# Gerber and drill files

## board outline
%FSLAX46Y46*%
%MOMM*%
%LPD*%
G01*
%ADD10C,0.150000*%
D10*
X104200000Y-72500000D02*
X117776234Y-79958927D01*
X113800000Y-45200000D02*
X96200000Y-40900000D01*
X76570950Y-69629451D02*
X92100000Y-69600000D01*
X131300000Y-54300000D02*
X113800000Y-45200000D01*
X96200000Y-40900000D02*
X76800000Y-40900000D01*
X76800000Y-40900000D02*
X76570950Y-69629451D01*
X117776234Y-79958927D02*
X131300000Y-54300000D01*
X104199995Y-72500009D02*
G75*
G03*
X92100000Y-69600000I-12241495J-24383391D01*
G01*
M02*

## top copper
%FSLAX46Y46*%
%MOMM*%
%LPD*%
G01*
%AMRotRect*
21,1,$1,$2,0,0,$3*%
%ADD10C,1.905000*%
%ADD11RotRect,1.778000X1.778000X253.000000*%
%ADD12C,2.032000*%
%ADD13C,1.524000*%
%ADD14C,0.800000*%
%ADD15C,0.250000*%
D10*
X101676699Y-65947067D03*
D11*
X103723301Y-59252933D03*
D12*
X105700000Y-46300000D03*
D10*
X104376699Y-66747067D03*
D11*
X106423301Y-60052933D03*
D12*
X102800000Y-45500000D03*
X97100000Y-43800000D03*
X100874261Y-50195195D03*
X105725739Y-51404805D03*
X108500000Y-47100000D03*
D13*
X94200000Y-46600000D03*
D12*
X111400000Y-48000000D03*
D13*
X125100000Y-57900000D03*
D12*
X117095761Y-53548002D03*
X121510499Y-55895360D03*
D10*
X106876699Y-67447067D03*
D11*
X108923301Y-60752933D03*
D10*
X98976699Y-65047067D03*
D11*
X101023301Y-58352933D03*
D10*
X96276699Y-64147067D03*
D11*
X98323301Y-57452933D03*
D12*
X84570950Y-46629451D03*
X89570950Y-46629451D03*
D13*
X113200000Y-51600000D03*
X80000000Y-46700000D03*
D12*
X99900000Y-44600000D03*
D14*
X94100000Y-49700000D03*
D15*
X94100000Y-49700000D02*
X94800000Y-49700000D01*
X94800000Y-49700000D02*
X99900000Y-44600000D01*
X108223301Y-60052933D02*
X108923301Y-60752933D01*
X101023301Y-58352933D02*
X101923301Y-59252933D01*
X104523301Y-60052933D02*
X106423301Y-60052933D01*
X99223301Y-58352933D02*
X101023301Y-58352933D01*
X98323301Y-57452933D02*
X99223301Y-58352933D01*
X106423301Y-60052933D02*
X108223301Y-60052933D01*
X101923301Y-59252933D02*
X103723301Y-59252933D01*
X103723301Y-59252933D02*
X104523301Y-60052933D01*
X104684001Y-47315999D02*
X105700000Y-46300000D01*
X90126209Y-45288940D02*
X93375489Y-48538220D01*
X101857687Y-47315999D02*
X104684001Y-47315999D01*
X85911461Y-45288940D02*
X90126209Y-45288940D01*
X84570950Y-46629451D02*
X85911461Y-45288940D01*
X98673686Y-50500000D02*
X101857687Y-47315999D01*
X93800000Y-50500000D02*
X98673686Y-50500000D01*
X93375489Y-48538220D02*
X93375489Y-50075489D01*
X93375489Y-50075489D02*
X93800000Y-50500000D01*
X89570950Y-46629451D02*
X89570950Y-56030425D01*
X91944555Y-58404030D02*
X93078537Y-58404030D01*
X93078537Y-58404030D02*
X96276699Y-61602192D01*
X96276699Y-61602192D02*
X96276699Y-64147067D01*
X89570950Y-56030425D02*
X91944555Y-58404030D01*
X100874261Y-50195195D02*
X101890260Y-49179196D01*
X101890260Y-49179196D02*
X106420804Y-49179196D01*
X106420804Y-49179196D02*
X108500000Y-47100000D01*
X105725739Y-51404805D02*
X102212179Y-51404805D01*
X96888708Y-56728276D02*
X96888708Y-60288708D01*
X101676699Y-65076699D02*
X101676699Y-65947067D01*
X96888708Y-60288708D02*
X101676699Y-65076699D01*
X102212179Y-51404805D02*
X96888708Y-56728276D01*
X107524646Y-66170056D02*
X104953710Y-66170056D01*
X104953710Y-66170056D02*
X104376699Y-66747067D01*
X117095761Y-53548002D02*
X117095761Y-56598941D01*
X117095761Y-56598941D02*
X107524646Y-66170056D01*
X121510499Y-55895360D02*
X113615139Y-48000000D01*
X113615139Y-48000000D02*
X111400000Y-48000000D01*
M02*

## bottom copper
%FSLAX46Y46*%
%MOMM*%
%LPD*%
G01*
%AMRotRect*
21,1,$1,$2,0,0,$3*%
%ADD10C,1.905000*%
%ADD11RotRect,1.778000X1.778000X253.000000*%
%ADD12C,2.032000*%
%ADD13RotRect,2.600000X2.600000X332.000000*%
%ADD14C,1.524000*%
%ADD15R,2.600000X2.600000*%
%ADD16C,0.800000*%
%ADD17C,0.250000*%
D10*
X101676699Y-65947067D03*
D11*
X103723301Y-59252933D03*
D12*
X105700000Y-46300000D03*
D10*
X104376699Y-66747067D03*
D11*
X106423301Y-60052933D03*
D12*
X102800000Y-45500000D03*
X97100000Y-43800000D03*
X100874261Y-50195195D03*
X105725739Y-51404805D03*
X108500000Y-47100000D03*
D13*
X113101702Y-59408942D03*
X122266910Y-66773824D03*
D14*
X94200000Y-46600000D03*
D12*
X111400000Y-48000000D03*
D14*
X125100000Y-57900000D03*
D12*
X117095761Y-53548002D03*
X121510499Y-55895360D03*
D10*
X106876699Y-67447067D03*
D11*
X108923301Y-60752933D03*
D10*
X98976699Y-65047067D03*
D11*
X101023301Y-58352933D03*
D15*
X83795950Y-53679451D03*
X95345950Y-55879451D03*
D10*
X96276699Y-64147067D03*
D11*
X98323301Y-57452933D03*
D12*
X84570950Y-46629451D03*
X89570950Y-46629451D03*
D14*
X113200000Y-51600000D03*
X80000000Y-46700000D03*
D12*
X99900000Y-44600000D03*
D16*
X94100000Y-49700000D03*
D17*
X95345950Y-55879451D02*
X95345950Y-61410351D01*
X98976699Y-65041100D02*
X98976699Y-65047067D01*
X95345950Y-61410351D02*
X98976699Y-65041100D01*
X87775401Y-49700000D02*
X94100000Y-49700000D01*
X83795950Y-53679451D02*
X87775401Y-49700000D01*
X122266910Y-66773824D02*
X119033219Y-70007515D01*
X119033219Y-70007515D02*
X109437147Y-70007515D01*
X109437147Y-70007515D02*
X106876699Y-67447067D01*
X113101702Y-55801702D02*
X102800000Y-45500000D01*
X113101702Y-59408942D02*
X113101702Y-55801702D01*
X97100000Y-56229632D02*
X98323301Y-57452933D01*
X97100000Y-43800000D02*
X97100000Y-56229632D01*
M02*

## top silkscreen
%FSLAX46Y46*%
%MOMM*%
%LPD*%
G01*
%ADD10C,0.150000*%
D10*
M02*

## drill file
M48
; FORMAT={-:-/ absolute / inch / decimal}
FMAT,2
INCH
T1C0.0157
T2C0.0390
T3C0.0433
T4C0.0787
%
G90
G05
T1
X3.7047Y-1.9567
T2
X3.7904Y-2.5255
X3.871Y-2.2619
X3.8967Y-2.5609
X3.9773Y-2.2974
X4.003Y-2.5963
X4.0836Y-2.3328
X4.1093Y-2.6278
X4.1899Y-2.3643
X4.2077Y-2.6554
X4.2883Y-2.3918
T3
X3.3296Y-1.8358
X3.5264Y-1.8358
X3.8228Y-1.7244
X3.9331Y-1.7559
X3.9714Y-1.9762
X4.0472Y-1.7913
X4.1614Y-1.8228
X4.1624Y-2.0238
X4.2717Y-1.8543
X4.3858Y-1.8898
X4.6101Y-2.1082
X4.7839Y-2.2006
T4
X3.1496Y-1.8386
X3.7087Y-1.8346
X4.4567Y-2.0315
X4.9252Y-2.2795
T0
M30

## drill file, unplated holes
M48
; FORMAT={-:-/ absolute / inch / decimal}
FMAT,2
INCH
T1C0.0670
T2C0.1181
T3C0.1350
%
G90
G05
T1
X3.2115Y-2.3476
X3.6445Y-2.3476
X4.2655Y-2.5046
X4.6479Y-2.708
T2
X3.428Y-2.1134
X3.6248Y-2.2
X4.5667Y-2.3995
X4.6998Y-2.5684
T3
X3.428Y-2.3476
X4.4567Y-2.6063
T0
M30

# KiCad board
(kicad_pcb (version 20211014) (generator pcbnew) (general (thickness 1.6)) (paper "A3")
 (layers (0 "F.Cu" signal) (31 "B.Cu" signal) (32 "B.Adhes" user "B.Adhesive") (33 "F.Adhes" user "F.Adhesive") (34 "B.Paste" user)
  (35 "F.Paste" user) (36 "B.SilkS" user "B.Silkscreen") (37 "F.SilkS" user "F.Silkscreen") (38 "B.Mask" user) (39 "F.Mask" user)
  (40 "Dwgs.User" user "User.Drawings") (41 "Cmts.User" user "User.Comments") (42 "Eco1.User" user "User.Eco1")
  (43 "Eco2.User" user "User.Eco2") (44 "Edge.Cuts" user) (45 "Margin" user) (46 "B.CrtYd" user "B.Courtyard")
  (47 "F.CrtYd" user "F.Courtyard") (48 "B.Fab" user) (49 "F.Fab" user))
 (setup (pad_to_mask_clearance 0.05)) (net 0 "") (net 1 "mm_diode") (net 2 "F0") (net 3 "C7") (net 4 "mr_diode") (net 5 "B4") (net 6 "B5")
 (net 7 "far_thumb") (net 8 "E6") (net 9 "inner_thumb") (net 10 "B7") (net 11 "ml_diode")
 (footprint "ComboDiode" (layer "F.Cu") (at 102.7 62.6 -107)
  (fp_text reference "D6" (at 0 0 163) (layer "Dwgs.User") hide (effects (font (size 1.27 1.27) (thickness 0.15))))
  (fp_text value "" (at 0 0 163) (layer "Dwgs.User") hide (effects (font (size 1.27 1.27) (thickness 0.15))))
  (pad "1" thru_hole circle locked (at 3.5 0 253) (size 1.905 1.905) (drill 0.9906) (layers *.Cu *.Mask) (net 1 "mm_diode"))
  (pad "2" thru_hole rect locked (at -3.5 0 253) (size 1.778 1.778) (drill 0.9906) (layers *.Cu *.Mask) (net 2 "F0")))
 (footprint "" (layer "F.Cu") (at 105.7 46.3)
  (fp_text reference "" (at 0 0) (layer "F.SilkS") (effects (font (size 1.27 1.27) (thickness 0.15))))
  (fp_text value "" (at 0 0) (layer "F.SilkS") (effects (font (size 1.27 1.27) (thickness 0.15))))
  (pad "1" thru_hole circle locked (at 0 0) (size 2.032 2.032) (drill 1.1) (layers *.Cu *.Mask) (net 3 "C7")))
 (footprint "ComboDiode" (layer "F.Cu") (at 105.4 63.4 -107)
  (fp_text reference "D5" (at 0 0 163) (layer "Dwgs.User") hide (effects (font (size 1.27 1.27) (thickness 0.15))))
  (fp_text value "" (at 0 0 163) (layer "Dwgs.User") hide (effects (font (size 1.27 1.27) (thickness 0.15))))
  (pad "1" thru_hole circle locked (at 3.5 0 253) (size 1.905 1.905) (drill 0.9906) (layers *.Cu *.Mask) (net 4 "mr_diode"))
  (pad "2" thru_hole rect locked (at -3.5 0 253) (size 1.778 1.778) (drill 0.9906) (layers *.Cu *.Mask) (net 2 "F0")))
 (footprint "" (layer "F.Cu") (at 102.8 45.5)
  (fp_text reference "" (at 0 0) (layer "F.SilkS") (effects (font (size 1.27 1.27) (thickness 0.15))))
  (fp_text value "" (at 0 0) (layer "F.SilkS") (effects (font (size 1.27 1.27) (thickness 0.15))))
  (pad "1" thru_hole circle locked (at 0 0) (size 2.032 2.032) (drill 1.1) (layers *.Cu *.Mask) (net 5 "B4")))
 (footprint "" (layer "F.Cu") (at 97.1 43.8)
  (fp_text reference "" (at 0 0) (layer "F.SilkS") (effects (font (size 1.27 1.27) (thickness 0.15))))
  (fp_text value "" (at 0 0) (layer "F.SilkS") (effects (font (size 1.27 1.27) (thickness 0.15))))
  (pad "1" thru_hole circle locked (at 0 0) (size 2.032 2.032) (drill 1.1) (layers *.Cu *.Mask) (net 2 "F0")))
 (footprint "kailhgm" (layer "F.Cu") (at 103.3 50.8 -14)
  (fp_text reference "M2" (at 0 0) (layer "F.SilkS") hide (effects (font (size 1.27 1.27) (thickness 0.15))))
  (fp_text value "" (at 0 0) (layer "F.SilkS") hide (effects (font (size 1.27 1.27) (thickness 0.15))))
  (pad "1" thru_hole circle locked (at -2.5 0) (size 2.032 2.032) (drill 1.1) (layers *.Cu *.Mask) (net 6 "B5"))
  (pad "2" thru_hole circle locked (at 2.5 0) (size 2.032 2.032) (drill 1.1) (layers *.Cu *.Mask) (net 1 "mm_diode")))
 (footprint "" (layer "F.Cu") (at 108.5 47.1)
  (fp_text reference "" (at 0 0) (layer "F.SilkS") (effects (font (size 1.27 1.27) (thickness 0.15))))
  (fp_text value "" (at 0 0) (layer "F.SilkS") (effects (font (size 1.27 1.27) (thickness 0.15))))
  (pad "1" thru_hole circle locked (at 0 0) (size 2.032 2.032) (drill 1.1) (layers *.Cu *.Mask) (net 6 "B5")))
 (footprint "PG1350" (layer "F.Cu") (at 113.2 66.2 -28)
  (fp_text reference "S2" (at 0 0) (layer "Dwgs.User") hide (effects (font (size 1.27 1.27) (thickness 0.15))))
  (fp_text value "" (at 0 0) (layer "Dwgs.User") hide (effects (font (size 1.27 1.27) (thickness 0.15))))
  (pad "" np_thru_hole circle locked (at 5 -3.75) (size 3 3) (drill 3) (layers *.Cu *.Mask))
  (pad "" np_thru_hole circle locked (at 5.5 0) (size 1.7018 1.7018) (drill 1.7018) (layers *.Cu *.Mask))
  (pad "" np_thru_hole circle locked (at 0 0) (size 3.429 3.429) (drill 3.429) (layers *.Cu *.Mask))
  (pad "" np_thru_hole circle locked (at -5.5 0) (size 1.7018 1.7018) (drill 1.7018) (layers *.Cu *.Mask))
  (pad "" np_thru_hole circle locked (at 0 -5.95) (size 3 3) (drill 3) (layers *.Cu *.Mask))
  (pad "1" smd rect locked (at -3.275 -5.95 332) (size 2.6 2.6) (layers "B.Cu" "B.Paste" "B.Mask") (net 5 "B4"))
  (pad "2" smd rect locked (at 8.275 -3.75 332) (size 2.6 2.6) (layers "B.Cu" "B.Paste" "B.Mask") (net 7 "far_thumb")))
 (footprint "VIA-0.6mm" (layer "F.Cu") (at 94.2 46.6)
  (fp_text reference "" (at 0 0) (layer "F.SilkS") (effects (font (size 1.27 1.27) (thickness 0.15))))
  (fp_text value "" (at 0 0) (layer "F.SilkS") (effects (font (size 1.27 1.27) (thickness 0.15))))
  (pad "1" thru_hole circle locked (at 0 0) (size 1.524 1.524) (drill 2) (layers *.Cu *.Mask)))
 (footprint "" (layer "F.Cu") (at 111.4 48)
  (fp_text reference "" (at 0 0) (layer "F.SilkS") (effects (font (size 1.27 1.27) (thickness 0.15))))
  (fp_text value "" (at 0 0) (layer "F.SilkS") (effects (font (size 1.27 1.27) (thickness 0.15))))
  (pad "1" thru_hole circle locked (at 0 0) (size 2.032 2.032) (drill 1.1) (layers *.Cu *.Mask) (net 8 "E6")))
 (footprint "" (layer "F.Cu") (at 125.1 57.9)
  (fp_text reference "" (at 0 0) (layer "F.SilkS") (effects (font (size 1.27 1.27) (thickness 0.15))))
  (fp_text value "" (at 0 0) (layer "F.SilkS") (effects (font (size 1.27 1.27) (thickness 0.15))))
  (pad "1" thru_hole circle locked (at 0 0) (size 1.524 1.524) (drill 2) (layers *.Cu *.Mask)))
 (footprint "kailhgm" (layer "F.Cu") (at 119.30313 54.721681 -28)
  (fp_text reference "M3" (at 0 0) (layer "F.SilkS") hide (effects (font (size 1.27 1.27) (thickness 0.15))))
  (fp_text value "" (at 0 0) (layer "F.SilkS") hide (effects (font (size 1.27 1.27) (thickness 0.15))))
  (pad "1" thru_hole circle locked (at -2.5 0) (size 2.032 2.032) (drill 1.1) (layers *.Cu *.Mask) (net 4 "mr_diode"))
  (pad "2" thru_hole circle locked (at 2.5 0) (size 2.032 2.032) (drill 1.1) (layers *.Cu *.Mask) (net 8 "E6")))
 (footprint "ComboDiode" (layer "F.Cu") (at 107.9 64.1 -107)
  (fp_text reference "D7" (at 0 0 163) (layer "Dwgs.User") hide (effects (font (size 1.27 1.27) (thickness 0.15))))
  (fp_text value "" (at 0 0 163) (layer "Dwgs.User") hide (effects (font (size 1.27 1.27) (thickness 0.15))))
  (pad "1" thru_hole circle locked (at 3.5 0 253) (size 1.905 1.905) (drill 0.9906) (layers *.Cu *.Mask) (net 7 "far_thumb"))
  (pad "2" thru_hole rect locked (at -3.5 0 253) (size 1.778 1.778) (drill 0.9906) (layers *.Cu *.Mask) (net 2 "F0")))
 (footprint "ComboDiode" (layer "F.Cu") (at 100 61.7 -107)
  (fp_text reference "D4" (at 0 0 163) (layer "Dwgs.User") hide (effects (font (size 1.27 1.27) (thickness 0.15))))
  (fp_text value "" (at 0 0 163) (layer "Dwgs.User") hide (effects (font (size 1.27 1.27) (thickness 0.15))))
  (pad "1" thru_hole circle locked (at 3.5 0 253) (size 1.905 1.905) (drill 0.9906) (layers *.Cu *.Mask) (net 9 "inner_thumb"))
  (pad "2" thru_hole rect locked (at -3.5 0 253) (size 1.778 1.778) (drill 0.9906) (layers *.Cu *.Mask) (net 2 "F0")))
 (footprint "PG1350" (layer "F.Cu") (at 87.07095 59.629451)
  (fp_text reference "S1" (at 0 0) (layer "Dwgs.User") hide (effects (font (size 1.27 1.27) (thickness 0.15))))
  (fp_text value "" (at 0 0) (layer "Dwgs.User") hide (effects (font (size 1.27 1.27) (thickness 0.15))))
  (pad "" np_thru_hole circle locked (at -5.5 0) (size 1.7018 1.7018) (drill 1.7018) (layers *.Cu *.Mask))
  (pad "" np_thru_hole circle locked (at 5 -3.75) (size 3 3) (drill 3) (layers *.Cu *.Mask))
  (pad "" np_thru_hole circle locked (at 5.5 0) (size 1.7018 1.7018) (drill 1.7018) (layers *.Cu *.Mask))
  (pad "" np_thru_hole circle locked (at 0 0) (size 3.429 3.429) (drill 3.429) (layers *.Cu *.Mask))
  (pad "" np_thru_hole circle locked (at 0 -5.95) (size 3 3) (drill 3) (layers *.Cu *.Mask))
  (pad "1" smd rect locked (at -3.275 -5.95) (size 2.6 2.6) (layers "B.Cu" "B.Paste" "B.Mask") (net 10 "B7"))
  (pad "2" smd rect locked (at 8.275 -3.75) (size 2.6 2.6) (layers "B.Cu" "B.Paste" "B.Mask") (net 9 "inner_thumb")))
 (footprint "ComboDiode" (layer "F.Cu") (at 97.3 60.8 -107)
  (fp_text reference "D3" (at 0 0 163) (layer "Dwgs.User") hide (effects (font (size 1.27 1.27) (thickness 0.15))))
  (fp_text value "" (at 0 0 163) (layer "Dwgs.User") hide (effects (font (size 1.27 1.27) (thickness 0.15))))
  (pad "1" thru_hole circle locked (at 3.5 0 253) (size 1.905 1.905) (drill 0.9906) (layers *.Cu *.Mask) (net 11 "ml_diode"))
  (pad "2" thru_hole rect locked (at -3.5 0 253) (size 1.778 1.778) (drill 0.9906) (layers *.Cu *.Mask) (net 2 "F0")))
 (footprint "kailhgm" (layer "F.Cu") (at 87.07095 46.629451)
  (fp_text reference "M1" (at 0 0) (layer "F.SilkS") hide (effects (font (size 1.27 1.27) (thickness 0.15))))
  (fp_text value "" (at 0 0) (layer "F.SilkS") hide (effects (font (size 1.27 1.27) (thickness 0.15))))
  (pad "1" thru_hole circle locked (at -2.5 0) (size 2.032 2.032) (drill 1.1) (layers *.Cu *.Mask) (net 3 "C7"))
  (pad "2" thru_hole circle locked (at 2.5 0) (size 2.032 2.032) (drill 1.1) (layers *.Cu *.Mask) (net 11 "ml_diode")))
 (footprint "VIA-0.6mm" (layer "F.Cu") (at 113.2 51.6 -28)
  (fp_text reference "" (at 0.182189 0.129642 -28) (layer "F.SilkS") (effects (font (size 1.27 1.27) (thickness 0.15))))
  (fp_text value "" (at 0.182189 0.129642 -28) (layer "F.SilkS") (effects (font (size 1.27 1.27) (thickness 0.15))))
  (pad "1" thru_hole circle locked (at 0 0) (size 1.524 1.524) (drill 2) (layers *.Cu *.Mask)))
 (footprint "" (layer "F.Cu") (at 80 46.7)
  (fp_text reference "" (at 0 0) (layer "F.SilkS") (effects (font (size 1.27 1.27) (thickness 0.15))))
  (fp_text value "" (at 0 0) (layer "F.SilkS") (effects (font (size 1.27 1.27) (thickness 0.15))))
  (pad "1" thru_hole circle locked (at 0 0) (size 1.524 1.524) (drill 2) (layers *.Cu *.Mask)))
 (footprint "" (layer "F.Cu") (at 99.9 44.6)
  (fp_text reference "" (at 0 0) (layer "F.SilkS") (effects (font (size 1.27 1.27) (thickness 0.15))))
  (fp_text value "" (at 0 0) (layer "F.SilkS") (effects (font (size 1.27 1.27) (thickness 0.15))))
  (pad "1" thru_hole circle locked (at 0 0) (size 2.032 2.032) (drill 1.1) (layers *.Cu *.Mask) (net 10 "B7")))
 (gr_line (start 104.2 72.5) (end 117.776234 79.958927) (layer "Edge.Cuts") (width 0.15))
 (gr_line (start 113.8 45.2) (end 96.2 40.9) (layer "Edge.Cuts") (width 0.15))
 (gr_line (start 76.57095 69.629451) (end 92.1 69.6) (layer "Edge.Cuts") (width 0.15))
 (gr_line (start 131.3 54.3) (end 113.8 45.2) (layer "Edge.Cuts") (width 0.15))
 (gr_line (start 96.2 40.9) (end 76.8 40.9) (layer "Edge.Cuts") (width 0.15))
 (gr_line (start 76.8 40.9) (end 76.57095 69.629451) (layer "Edge.Cuts") (width 0.15))
 (gr_line (start 117.776234 79.958927) (end 131.3 54.3) (layer "Edge.Cuts") (width 0.15))
 (gr_arc (start 92.1 69.6) (mid 98.317524 70.351024) (end 104.2 72.5) (layer "Edge.Cuts") (width 0.15))
 (segment (start 95.34595 55.879451) (end 95.34595 61.410351) (width 0.25) (layer "B.Cu") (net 9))
 (segment (start 98.976699 65.0411) (end 98.976699 65.047067) (width 0.25) (layer "B.Cu") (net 9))
 (segment (start 95.34595 61.410351) (end 98.976699 65.0411) (width 0.25) (layer "B.Cu") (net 9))
 (segment (start 94.1 49.7) (end 94.8 49.7) (width 0.25) (layer "F.Cu") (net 10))
 (segment (start 94.8 49.7) (end 99.9 44.6) (width 0.25) (layer "F.Cu") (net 10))
 (via (at 94.1 49.7) (size 0.8) (drill 0.4) (layers "F.Cu" "B.Cu") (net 10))
 (segment (start 87.775401 49.7) (end 94.1 49.7) (width 0.25) (layer "B.Cu") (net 10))
 (segment (start 83.79595 53.679451) (end 87.775401 49.7) (width 0.25) (layer "B.Cu") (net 10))
 (segment (start 122.26691 66.773824) (end 119.033219 70.007515) (width 0.25) (layer "B.Cu") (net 7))
 (segment (start 119.033219 70.007515) (end 109.437147 70.007515) (width 0.25) (layer "B.Cu") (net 7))
 (segment (start 109.437147 70.007515) (end 106.876699 67.447067) (width 0.25) (layer "B.Cu") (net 7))
 (segment (start 113.101702 55.801702) (end 102.8 45.5) (width 0.25) (layer "B.Cu") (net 5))
 (segment (start 113.101702 59.408942) (end 113.101702 55.801702) (width 0.25) (layer "B.Cu") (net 5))
 (segment (start 108.223301 60.052933) (end 108.923301 60.752933) (width 0.25) (layer "F.Cu") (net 2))
 (segment (start 101.023301 58.352933) (end 101.923301 59.252933) (width 0.25) (layer "F.Cu") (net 2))
 (segment (start 104.523301 60.052933) (end 106.423301 60.052933) (width 0.25) (layer "F.Cu") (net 2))
 (segment (start 99.223301 58.352933) (end 101.023301 58.352933) (width 0.25) (layer "F.Cu") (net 2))
 (segment (start 98.323301 57.452933) (end 99.223301 58.352933) (width 0.25) (layer "F.Cu") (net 2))
 (segment (start 106.423301 60.052933) (end 108.223301 60.052933) (width 0.25) (layer "F.Cu") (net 2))
 (segment (start 101.923301 59.252933) (end 103.723301 59.252933) (width 0.25) (layer "F.Cu") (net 2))
 (segment (start 103.723301 59.252933) (end 104.523301 60.052933) (width 0.25) (layer "F.Cu") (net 2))
 (segment (start 97.1 56.229632) (end 98.323301 57.452933) (width 0.25) (layer "B.Cu") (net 2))
 (segment (start 97.1 43.8) (end 97.1 56.229632) (width 0.25) (layer "B.Cu") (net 2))
 (segment (start 104.684001 47.315999) (end 105.7 46.3) (width 0.25) (layer "F.Cu") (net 3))
 (segment (start 90.126209 45.28894) (end 93.375489 48.53822) (width 0.25) (layer "F.Cu") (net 3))
 (segment (start 101.857687 47.315999) (end 104.684001 47.315999) (width 0.25) (layer "F.Cu") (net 3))
 (segment (start 85.911461 45.28894) (end 90.126209 45.28894) (width 0.25) (layer "F.Cu") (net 3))
 (segment (start 84.57095 46.629451) (end 85.911461 45.28894) (width 0.25) (layer "F.Cu") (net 3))
 (segment (start 98.673686 50.5) (end 101.857687 47.315999) (width 0.25) (layer "F.Cu") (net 3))
 (segment (start 93.8 50.5) (end 98.673686 50.5) (width 0.25) (layer "F.Cu") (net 3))
 (segment (start 93.375489 48.53822) (end 93.375489 50.075489) (width 0.25) (layer "F.Cu") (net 3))
 (segment (start 93.375489 50.075489) (end 93.8 50.5) (width 0.25) (layer "F.Cu") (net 3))
 (segment (start 89.57095 46.629451) (end 89.57095 56.030425) (width 0.25) (layer "F.Cu") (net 11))
 (segment (start 91.944555 58.40403) (end 93.078537 58.40403) (width 0.25) (layer "F.Cu") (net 11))
 (segment (start 93.078537 58.40403) (end 96.276699 61.602192) (width 0.25) (layer "F.Cu") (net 11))
 (segment (start 96.276699 61.602192) (end 96.276699 64.147067) (width 0.25) (layer "F.Cu") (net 11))
 (segment (start 89.57095 56.030425) (end 91.944555 58.40403) (width 0.25) (layer "F.Cu") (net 11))
 (segment (start 100.874261 50.195195) (end 101.89026 49.179196) (width 0.25) (layer "F.Cu") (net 6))
 (segment (start 101.89026 49.179196) (end 106.420804 49.179196) (width 0.25) (layer "F.Cu") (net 6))
 (segment (start 106.420804 49.179196) (end 108.5 47.1) (width 0.25) (layer "F.Cu") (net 6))
 (segment (start 105.725739 51.404805) (end 102.212179 51.404805) (width 0.25) (layer "F.Cu") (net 1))
 (segment (start 96.888708 56.728276) (end 96.888708 60.288708) (width 0.25) (layer "F.Cu") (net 1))
 (segment (start 101.676699 65.076699) (end 101.676699 65.947067) (width 0.25) (layer "F.Cu") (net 1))
 (segment (start 96.888708 60.288708) (end 101.676699 65.076699) (width 0.25) (layer "F.Cu") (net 1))
 (segment (start 102.212179 51.404805) (end 96.888708 56.728276) (width 0.25) (layer "F.Cu") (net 1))
 (segment (start 107.524646 66.170056) (end 104.95371 66.170056) (width 0.25) (layer "F.Cu") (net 4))
 (segment (start 104.95371 66.170056) (end 104.376699 66.747067) (width 0.25) (layer "F.Cu") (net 4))
 (segment (start 117.095761 53.548002) (end 117.095761 56.598941) (width 0.25) (layer "F.Cu") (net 4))
 (segment (start 117.095761 56.598941) (end 107.524646 66.170056) (width 0.25) (layer "F.Cu") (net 4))
 (segment (start 121.510499 55.89536) (end 113.615139 48) (width 0.25) (layer "F.Cu") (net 8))
 (segment (start 113.615139 48) (end 111.4 48) (width 0.25) (layer "F.Cu") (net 8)))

